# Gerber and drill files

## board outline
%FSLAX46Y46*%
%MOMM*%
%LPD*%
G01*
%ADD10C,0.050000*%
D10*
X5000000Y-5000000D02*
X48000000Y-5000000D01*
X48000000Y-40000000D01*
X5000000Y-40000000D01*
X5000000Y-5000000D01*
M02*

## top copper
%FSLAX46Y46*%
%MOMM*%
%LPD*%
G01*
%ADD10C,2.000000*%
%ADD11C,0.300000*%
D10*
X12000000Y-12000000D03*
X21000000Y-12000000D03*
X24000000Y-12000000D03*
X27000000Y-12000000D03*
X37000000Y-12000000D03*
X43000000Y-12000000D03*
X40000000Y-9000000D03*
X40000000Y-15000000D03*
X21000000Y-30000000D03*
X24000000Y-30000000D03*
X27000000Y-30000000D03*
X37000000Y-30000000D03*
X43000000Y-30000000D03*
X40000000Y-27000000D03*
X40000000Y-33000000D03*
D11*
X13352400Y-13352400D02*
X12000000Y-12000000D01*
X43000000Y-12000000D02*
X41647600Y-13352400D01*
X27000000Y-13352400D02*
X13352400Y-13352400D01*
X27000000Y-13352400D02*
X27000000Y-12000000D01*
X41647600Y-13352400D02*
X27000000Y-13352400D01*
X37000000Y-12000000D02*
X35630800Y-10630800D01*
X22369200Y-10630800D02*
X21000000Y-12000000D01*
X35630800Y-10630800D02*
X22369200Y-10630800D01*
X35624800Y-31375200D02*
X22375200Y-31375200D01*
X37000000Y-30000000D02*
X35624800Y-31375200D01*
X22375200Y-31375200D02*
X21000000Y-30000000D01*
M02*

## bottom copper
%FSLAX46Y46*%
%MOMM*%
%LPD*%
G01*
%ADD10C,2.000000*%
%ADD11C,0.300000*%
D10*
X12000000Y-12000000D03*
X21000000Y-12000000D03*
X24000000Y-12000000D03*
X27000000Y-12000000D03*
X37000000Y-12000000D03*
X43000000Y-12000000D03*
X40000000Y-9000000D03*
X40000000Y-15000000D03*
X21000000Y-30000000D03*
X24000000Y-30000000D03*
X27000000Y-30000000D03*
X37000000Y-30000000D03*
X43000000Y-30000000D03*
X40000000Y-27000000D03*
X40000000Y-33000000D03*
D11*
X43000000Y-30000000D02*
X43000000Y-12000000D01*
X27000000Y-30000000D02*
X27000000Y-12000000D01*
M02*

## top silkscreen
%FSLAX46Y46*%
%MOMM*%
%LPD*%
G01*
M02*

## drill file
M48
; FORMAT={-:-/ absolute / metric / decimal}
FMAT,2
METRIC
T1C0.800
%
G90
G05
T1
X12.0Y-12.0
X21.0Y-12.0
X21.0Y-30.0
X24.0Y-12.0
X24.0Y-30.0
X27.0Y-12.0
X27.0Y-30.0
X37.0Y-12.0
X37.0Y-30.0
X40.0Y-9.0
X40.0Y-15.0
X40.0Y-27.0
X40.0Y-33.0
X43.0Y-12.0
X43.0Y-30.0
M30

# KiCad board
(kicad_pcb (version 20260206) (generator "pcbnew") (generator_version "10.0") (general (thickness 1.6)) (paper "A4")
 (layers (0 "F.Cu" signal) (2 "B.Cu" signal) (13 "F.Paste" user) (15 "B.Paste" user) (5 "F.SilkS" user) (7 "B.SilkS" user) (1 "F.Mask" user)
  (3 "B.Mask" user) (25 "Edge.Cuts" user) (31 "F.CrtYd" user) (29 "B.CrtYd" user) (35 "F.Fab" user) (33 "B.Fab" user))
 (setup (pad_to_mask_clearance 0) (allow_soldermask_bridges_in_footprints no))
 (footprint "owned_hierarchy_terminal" (layer "F.Cu") (at 12 12)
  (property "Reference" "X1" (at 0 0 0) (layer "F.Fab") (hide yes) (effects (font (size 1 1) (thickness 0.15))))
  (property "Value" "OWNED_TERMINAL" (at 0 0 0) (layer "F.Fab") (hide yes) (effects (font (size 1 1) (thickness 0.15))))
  (pad "1" thru_hole circle (at 0 0) (size 2 2) (drill 0.8) (layers "*.Cu" "*.Mask") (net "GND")))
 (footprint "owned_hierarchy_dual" (layer "F.Cu") (at 24 12)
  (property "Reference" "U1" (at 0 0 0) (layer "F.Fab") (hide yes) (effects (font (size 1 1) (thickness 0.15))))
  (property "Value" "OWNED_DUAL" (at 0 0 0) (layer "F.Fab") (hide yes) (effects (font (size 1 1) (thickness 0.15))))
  (pad "1" thru_hole circle (at -3 0) (size 2 2) (drill 0.8) (layers "*.Cu" "*.Mask") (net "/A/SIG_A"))
  (pad "2" thru_hole circle (at 0 0) (size 2 2) (drill 0.8) (layers "*.Cu" "*.Mask") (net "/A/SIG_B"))
  (pad "3" thru_hole circle (at 3 0) (size 2 2) (drill 0.8) (layers "*.Cu" "*.Mask") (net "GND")))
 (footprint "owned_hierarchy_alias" (layer "F.Cu") (at 40 12)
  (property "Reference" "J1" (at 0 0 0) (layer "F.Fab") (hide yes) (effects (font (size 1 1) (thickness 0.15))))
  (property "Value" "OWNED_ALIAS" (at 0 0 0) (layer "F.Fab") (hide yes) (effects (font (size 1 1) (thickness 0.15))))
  (pad "R" thru_hole circle (at -3 0) (size 2 2) (drill 0.8) (layers "*.Cu" "*.Mask") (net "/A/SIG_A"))
  (pad "T" thru_hole circle (at 3 0) (size 2 2) (drill 0.8) (layers "*.Cu" "*.Mask") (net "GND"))
  (pad "MP" thru_hole circle (at 0 -3) (size 2 2) (drill 0.8) (layers "*.Cu" "*.Mask"))
  (pad "MP" thru_hole circle (at 0 3) (size 2 2) (drill 0.8) (layers "*.Cu" "*.Mask")))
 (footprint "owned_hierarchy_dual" (layer "F.Cu") (at 24 30)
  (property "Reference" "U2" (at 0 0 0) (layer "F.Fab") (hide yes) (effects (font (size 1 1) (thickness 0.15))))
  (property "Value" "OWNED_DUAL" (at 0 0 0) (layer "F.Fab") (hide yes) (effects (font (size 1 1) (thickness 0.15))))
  (pad "1" thru_hole circle (at -3 0) (size 2 2) (drill 0.8) (layers "*.Cu" "*.Mask") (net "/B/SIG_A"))
  (pad "2" thru_hole circle (at 0 0) (size 2 2) (drill 0.8) (layers "*.Cu" "*.Mask") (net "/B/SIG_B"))
  (pad "3" thru_hole circle (at 3 0) (size 2 2) (drill 0.8) (layers "*.Cu" "*.Mask") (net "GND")))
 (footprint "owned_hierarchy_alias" (layer "F.Cu") (at 40 30)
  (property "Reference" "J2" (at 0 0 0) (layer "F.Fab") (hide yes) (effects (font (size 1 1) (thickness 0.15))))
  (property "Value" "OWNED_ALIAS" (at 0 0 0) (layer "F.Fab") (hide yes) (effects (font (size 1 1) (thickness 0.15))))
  (pad "R" thru_hole circle (at -3 0) (size 2 2) (drill 0.8) (layers "*.Cu" "*.Mask") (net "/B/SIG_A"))
  (pad "T" thru_hole circle (at 3 0) (size 2 2) (drill 0.8) (layers "*.Cu" "*.Mask") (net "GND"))
  (pad "MP" thru_hole circle (at 0 -3) (size 2 2) (drill 0.8) (layers "*.Cu" "*.Mask"))
  (pad "MP" thru_hole circle (at 0 3) (size 2 2) (drill 0.8) (layers "*.Cu" "*.Mask")))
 (gr_rect (start 5 5) (end 48 40) (stroke (width 0.05) (type default)) (fill none) (layer "Edge.Cuts"))
 (segment (start 13.3524 13.3524) (end 12 12) (width 0.3) (layer "F.Cu") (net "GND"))
 (segment (start 43 12) (end 41.6476 13.3524) (width 0.3) (layer "F.Cu") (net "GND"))
 (segment (start 27 13.3524) (end 13.3524 13.3524) (width 0.3) (layer "F.Cu") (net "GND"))
 (segment (start 27 13.3524) (end 27 12) (width 0.3) (layer "F.Cu") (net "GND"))
 (segment (start 41.6476 13.3524) (end 27 13.3524) (width 0.3) (layer "F.Cu") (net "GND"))
 (segment (start 43 30) (end 43 12) (width 0.3) (layer "B.Cu") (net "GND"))
 (segment (start 27 30) (end 27 12) (width 0.3) (layer "B.Cu") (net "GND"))
 (segment (start 37 12) (end 35.6308 10.6308) (width 0.3) (layer "F.Cu") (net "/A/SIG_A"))
 (segment (start 22.3692 10.6308) (end 21 12) (width 0.3) (layer "F.Cu") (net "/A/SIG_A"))
 (segment (start 35.6308 10.6308) (end 22.3692 10.6308) (width 0.3) (layer "F.Cu") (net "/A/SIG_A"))
 (segment (start 35.6248 31.3752) (end 22.3752 31.3752) (width 0.3) (layer "F.Cu") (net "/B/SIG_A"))
 (segment (start 37 30) (end 35.6248 31.3752) (width 0.3) (layer "F.Cu") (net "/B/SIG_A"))
 (segment (start 22.3752 31.3752) (end 21 30) (width 0.3) (layer "F.Cu") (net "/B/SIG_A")))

